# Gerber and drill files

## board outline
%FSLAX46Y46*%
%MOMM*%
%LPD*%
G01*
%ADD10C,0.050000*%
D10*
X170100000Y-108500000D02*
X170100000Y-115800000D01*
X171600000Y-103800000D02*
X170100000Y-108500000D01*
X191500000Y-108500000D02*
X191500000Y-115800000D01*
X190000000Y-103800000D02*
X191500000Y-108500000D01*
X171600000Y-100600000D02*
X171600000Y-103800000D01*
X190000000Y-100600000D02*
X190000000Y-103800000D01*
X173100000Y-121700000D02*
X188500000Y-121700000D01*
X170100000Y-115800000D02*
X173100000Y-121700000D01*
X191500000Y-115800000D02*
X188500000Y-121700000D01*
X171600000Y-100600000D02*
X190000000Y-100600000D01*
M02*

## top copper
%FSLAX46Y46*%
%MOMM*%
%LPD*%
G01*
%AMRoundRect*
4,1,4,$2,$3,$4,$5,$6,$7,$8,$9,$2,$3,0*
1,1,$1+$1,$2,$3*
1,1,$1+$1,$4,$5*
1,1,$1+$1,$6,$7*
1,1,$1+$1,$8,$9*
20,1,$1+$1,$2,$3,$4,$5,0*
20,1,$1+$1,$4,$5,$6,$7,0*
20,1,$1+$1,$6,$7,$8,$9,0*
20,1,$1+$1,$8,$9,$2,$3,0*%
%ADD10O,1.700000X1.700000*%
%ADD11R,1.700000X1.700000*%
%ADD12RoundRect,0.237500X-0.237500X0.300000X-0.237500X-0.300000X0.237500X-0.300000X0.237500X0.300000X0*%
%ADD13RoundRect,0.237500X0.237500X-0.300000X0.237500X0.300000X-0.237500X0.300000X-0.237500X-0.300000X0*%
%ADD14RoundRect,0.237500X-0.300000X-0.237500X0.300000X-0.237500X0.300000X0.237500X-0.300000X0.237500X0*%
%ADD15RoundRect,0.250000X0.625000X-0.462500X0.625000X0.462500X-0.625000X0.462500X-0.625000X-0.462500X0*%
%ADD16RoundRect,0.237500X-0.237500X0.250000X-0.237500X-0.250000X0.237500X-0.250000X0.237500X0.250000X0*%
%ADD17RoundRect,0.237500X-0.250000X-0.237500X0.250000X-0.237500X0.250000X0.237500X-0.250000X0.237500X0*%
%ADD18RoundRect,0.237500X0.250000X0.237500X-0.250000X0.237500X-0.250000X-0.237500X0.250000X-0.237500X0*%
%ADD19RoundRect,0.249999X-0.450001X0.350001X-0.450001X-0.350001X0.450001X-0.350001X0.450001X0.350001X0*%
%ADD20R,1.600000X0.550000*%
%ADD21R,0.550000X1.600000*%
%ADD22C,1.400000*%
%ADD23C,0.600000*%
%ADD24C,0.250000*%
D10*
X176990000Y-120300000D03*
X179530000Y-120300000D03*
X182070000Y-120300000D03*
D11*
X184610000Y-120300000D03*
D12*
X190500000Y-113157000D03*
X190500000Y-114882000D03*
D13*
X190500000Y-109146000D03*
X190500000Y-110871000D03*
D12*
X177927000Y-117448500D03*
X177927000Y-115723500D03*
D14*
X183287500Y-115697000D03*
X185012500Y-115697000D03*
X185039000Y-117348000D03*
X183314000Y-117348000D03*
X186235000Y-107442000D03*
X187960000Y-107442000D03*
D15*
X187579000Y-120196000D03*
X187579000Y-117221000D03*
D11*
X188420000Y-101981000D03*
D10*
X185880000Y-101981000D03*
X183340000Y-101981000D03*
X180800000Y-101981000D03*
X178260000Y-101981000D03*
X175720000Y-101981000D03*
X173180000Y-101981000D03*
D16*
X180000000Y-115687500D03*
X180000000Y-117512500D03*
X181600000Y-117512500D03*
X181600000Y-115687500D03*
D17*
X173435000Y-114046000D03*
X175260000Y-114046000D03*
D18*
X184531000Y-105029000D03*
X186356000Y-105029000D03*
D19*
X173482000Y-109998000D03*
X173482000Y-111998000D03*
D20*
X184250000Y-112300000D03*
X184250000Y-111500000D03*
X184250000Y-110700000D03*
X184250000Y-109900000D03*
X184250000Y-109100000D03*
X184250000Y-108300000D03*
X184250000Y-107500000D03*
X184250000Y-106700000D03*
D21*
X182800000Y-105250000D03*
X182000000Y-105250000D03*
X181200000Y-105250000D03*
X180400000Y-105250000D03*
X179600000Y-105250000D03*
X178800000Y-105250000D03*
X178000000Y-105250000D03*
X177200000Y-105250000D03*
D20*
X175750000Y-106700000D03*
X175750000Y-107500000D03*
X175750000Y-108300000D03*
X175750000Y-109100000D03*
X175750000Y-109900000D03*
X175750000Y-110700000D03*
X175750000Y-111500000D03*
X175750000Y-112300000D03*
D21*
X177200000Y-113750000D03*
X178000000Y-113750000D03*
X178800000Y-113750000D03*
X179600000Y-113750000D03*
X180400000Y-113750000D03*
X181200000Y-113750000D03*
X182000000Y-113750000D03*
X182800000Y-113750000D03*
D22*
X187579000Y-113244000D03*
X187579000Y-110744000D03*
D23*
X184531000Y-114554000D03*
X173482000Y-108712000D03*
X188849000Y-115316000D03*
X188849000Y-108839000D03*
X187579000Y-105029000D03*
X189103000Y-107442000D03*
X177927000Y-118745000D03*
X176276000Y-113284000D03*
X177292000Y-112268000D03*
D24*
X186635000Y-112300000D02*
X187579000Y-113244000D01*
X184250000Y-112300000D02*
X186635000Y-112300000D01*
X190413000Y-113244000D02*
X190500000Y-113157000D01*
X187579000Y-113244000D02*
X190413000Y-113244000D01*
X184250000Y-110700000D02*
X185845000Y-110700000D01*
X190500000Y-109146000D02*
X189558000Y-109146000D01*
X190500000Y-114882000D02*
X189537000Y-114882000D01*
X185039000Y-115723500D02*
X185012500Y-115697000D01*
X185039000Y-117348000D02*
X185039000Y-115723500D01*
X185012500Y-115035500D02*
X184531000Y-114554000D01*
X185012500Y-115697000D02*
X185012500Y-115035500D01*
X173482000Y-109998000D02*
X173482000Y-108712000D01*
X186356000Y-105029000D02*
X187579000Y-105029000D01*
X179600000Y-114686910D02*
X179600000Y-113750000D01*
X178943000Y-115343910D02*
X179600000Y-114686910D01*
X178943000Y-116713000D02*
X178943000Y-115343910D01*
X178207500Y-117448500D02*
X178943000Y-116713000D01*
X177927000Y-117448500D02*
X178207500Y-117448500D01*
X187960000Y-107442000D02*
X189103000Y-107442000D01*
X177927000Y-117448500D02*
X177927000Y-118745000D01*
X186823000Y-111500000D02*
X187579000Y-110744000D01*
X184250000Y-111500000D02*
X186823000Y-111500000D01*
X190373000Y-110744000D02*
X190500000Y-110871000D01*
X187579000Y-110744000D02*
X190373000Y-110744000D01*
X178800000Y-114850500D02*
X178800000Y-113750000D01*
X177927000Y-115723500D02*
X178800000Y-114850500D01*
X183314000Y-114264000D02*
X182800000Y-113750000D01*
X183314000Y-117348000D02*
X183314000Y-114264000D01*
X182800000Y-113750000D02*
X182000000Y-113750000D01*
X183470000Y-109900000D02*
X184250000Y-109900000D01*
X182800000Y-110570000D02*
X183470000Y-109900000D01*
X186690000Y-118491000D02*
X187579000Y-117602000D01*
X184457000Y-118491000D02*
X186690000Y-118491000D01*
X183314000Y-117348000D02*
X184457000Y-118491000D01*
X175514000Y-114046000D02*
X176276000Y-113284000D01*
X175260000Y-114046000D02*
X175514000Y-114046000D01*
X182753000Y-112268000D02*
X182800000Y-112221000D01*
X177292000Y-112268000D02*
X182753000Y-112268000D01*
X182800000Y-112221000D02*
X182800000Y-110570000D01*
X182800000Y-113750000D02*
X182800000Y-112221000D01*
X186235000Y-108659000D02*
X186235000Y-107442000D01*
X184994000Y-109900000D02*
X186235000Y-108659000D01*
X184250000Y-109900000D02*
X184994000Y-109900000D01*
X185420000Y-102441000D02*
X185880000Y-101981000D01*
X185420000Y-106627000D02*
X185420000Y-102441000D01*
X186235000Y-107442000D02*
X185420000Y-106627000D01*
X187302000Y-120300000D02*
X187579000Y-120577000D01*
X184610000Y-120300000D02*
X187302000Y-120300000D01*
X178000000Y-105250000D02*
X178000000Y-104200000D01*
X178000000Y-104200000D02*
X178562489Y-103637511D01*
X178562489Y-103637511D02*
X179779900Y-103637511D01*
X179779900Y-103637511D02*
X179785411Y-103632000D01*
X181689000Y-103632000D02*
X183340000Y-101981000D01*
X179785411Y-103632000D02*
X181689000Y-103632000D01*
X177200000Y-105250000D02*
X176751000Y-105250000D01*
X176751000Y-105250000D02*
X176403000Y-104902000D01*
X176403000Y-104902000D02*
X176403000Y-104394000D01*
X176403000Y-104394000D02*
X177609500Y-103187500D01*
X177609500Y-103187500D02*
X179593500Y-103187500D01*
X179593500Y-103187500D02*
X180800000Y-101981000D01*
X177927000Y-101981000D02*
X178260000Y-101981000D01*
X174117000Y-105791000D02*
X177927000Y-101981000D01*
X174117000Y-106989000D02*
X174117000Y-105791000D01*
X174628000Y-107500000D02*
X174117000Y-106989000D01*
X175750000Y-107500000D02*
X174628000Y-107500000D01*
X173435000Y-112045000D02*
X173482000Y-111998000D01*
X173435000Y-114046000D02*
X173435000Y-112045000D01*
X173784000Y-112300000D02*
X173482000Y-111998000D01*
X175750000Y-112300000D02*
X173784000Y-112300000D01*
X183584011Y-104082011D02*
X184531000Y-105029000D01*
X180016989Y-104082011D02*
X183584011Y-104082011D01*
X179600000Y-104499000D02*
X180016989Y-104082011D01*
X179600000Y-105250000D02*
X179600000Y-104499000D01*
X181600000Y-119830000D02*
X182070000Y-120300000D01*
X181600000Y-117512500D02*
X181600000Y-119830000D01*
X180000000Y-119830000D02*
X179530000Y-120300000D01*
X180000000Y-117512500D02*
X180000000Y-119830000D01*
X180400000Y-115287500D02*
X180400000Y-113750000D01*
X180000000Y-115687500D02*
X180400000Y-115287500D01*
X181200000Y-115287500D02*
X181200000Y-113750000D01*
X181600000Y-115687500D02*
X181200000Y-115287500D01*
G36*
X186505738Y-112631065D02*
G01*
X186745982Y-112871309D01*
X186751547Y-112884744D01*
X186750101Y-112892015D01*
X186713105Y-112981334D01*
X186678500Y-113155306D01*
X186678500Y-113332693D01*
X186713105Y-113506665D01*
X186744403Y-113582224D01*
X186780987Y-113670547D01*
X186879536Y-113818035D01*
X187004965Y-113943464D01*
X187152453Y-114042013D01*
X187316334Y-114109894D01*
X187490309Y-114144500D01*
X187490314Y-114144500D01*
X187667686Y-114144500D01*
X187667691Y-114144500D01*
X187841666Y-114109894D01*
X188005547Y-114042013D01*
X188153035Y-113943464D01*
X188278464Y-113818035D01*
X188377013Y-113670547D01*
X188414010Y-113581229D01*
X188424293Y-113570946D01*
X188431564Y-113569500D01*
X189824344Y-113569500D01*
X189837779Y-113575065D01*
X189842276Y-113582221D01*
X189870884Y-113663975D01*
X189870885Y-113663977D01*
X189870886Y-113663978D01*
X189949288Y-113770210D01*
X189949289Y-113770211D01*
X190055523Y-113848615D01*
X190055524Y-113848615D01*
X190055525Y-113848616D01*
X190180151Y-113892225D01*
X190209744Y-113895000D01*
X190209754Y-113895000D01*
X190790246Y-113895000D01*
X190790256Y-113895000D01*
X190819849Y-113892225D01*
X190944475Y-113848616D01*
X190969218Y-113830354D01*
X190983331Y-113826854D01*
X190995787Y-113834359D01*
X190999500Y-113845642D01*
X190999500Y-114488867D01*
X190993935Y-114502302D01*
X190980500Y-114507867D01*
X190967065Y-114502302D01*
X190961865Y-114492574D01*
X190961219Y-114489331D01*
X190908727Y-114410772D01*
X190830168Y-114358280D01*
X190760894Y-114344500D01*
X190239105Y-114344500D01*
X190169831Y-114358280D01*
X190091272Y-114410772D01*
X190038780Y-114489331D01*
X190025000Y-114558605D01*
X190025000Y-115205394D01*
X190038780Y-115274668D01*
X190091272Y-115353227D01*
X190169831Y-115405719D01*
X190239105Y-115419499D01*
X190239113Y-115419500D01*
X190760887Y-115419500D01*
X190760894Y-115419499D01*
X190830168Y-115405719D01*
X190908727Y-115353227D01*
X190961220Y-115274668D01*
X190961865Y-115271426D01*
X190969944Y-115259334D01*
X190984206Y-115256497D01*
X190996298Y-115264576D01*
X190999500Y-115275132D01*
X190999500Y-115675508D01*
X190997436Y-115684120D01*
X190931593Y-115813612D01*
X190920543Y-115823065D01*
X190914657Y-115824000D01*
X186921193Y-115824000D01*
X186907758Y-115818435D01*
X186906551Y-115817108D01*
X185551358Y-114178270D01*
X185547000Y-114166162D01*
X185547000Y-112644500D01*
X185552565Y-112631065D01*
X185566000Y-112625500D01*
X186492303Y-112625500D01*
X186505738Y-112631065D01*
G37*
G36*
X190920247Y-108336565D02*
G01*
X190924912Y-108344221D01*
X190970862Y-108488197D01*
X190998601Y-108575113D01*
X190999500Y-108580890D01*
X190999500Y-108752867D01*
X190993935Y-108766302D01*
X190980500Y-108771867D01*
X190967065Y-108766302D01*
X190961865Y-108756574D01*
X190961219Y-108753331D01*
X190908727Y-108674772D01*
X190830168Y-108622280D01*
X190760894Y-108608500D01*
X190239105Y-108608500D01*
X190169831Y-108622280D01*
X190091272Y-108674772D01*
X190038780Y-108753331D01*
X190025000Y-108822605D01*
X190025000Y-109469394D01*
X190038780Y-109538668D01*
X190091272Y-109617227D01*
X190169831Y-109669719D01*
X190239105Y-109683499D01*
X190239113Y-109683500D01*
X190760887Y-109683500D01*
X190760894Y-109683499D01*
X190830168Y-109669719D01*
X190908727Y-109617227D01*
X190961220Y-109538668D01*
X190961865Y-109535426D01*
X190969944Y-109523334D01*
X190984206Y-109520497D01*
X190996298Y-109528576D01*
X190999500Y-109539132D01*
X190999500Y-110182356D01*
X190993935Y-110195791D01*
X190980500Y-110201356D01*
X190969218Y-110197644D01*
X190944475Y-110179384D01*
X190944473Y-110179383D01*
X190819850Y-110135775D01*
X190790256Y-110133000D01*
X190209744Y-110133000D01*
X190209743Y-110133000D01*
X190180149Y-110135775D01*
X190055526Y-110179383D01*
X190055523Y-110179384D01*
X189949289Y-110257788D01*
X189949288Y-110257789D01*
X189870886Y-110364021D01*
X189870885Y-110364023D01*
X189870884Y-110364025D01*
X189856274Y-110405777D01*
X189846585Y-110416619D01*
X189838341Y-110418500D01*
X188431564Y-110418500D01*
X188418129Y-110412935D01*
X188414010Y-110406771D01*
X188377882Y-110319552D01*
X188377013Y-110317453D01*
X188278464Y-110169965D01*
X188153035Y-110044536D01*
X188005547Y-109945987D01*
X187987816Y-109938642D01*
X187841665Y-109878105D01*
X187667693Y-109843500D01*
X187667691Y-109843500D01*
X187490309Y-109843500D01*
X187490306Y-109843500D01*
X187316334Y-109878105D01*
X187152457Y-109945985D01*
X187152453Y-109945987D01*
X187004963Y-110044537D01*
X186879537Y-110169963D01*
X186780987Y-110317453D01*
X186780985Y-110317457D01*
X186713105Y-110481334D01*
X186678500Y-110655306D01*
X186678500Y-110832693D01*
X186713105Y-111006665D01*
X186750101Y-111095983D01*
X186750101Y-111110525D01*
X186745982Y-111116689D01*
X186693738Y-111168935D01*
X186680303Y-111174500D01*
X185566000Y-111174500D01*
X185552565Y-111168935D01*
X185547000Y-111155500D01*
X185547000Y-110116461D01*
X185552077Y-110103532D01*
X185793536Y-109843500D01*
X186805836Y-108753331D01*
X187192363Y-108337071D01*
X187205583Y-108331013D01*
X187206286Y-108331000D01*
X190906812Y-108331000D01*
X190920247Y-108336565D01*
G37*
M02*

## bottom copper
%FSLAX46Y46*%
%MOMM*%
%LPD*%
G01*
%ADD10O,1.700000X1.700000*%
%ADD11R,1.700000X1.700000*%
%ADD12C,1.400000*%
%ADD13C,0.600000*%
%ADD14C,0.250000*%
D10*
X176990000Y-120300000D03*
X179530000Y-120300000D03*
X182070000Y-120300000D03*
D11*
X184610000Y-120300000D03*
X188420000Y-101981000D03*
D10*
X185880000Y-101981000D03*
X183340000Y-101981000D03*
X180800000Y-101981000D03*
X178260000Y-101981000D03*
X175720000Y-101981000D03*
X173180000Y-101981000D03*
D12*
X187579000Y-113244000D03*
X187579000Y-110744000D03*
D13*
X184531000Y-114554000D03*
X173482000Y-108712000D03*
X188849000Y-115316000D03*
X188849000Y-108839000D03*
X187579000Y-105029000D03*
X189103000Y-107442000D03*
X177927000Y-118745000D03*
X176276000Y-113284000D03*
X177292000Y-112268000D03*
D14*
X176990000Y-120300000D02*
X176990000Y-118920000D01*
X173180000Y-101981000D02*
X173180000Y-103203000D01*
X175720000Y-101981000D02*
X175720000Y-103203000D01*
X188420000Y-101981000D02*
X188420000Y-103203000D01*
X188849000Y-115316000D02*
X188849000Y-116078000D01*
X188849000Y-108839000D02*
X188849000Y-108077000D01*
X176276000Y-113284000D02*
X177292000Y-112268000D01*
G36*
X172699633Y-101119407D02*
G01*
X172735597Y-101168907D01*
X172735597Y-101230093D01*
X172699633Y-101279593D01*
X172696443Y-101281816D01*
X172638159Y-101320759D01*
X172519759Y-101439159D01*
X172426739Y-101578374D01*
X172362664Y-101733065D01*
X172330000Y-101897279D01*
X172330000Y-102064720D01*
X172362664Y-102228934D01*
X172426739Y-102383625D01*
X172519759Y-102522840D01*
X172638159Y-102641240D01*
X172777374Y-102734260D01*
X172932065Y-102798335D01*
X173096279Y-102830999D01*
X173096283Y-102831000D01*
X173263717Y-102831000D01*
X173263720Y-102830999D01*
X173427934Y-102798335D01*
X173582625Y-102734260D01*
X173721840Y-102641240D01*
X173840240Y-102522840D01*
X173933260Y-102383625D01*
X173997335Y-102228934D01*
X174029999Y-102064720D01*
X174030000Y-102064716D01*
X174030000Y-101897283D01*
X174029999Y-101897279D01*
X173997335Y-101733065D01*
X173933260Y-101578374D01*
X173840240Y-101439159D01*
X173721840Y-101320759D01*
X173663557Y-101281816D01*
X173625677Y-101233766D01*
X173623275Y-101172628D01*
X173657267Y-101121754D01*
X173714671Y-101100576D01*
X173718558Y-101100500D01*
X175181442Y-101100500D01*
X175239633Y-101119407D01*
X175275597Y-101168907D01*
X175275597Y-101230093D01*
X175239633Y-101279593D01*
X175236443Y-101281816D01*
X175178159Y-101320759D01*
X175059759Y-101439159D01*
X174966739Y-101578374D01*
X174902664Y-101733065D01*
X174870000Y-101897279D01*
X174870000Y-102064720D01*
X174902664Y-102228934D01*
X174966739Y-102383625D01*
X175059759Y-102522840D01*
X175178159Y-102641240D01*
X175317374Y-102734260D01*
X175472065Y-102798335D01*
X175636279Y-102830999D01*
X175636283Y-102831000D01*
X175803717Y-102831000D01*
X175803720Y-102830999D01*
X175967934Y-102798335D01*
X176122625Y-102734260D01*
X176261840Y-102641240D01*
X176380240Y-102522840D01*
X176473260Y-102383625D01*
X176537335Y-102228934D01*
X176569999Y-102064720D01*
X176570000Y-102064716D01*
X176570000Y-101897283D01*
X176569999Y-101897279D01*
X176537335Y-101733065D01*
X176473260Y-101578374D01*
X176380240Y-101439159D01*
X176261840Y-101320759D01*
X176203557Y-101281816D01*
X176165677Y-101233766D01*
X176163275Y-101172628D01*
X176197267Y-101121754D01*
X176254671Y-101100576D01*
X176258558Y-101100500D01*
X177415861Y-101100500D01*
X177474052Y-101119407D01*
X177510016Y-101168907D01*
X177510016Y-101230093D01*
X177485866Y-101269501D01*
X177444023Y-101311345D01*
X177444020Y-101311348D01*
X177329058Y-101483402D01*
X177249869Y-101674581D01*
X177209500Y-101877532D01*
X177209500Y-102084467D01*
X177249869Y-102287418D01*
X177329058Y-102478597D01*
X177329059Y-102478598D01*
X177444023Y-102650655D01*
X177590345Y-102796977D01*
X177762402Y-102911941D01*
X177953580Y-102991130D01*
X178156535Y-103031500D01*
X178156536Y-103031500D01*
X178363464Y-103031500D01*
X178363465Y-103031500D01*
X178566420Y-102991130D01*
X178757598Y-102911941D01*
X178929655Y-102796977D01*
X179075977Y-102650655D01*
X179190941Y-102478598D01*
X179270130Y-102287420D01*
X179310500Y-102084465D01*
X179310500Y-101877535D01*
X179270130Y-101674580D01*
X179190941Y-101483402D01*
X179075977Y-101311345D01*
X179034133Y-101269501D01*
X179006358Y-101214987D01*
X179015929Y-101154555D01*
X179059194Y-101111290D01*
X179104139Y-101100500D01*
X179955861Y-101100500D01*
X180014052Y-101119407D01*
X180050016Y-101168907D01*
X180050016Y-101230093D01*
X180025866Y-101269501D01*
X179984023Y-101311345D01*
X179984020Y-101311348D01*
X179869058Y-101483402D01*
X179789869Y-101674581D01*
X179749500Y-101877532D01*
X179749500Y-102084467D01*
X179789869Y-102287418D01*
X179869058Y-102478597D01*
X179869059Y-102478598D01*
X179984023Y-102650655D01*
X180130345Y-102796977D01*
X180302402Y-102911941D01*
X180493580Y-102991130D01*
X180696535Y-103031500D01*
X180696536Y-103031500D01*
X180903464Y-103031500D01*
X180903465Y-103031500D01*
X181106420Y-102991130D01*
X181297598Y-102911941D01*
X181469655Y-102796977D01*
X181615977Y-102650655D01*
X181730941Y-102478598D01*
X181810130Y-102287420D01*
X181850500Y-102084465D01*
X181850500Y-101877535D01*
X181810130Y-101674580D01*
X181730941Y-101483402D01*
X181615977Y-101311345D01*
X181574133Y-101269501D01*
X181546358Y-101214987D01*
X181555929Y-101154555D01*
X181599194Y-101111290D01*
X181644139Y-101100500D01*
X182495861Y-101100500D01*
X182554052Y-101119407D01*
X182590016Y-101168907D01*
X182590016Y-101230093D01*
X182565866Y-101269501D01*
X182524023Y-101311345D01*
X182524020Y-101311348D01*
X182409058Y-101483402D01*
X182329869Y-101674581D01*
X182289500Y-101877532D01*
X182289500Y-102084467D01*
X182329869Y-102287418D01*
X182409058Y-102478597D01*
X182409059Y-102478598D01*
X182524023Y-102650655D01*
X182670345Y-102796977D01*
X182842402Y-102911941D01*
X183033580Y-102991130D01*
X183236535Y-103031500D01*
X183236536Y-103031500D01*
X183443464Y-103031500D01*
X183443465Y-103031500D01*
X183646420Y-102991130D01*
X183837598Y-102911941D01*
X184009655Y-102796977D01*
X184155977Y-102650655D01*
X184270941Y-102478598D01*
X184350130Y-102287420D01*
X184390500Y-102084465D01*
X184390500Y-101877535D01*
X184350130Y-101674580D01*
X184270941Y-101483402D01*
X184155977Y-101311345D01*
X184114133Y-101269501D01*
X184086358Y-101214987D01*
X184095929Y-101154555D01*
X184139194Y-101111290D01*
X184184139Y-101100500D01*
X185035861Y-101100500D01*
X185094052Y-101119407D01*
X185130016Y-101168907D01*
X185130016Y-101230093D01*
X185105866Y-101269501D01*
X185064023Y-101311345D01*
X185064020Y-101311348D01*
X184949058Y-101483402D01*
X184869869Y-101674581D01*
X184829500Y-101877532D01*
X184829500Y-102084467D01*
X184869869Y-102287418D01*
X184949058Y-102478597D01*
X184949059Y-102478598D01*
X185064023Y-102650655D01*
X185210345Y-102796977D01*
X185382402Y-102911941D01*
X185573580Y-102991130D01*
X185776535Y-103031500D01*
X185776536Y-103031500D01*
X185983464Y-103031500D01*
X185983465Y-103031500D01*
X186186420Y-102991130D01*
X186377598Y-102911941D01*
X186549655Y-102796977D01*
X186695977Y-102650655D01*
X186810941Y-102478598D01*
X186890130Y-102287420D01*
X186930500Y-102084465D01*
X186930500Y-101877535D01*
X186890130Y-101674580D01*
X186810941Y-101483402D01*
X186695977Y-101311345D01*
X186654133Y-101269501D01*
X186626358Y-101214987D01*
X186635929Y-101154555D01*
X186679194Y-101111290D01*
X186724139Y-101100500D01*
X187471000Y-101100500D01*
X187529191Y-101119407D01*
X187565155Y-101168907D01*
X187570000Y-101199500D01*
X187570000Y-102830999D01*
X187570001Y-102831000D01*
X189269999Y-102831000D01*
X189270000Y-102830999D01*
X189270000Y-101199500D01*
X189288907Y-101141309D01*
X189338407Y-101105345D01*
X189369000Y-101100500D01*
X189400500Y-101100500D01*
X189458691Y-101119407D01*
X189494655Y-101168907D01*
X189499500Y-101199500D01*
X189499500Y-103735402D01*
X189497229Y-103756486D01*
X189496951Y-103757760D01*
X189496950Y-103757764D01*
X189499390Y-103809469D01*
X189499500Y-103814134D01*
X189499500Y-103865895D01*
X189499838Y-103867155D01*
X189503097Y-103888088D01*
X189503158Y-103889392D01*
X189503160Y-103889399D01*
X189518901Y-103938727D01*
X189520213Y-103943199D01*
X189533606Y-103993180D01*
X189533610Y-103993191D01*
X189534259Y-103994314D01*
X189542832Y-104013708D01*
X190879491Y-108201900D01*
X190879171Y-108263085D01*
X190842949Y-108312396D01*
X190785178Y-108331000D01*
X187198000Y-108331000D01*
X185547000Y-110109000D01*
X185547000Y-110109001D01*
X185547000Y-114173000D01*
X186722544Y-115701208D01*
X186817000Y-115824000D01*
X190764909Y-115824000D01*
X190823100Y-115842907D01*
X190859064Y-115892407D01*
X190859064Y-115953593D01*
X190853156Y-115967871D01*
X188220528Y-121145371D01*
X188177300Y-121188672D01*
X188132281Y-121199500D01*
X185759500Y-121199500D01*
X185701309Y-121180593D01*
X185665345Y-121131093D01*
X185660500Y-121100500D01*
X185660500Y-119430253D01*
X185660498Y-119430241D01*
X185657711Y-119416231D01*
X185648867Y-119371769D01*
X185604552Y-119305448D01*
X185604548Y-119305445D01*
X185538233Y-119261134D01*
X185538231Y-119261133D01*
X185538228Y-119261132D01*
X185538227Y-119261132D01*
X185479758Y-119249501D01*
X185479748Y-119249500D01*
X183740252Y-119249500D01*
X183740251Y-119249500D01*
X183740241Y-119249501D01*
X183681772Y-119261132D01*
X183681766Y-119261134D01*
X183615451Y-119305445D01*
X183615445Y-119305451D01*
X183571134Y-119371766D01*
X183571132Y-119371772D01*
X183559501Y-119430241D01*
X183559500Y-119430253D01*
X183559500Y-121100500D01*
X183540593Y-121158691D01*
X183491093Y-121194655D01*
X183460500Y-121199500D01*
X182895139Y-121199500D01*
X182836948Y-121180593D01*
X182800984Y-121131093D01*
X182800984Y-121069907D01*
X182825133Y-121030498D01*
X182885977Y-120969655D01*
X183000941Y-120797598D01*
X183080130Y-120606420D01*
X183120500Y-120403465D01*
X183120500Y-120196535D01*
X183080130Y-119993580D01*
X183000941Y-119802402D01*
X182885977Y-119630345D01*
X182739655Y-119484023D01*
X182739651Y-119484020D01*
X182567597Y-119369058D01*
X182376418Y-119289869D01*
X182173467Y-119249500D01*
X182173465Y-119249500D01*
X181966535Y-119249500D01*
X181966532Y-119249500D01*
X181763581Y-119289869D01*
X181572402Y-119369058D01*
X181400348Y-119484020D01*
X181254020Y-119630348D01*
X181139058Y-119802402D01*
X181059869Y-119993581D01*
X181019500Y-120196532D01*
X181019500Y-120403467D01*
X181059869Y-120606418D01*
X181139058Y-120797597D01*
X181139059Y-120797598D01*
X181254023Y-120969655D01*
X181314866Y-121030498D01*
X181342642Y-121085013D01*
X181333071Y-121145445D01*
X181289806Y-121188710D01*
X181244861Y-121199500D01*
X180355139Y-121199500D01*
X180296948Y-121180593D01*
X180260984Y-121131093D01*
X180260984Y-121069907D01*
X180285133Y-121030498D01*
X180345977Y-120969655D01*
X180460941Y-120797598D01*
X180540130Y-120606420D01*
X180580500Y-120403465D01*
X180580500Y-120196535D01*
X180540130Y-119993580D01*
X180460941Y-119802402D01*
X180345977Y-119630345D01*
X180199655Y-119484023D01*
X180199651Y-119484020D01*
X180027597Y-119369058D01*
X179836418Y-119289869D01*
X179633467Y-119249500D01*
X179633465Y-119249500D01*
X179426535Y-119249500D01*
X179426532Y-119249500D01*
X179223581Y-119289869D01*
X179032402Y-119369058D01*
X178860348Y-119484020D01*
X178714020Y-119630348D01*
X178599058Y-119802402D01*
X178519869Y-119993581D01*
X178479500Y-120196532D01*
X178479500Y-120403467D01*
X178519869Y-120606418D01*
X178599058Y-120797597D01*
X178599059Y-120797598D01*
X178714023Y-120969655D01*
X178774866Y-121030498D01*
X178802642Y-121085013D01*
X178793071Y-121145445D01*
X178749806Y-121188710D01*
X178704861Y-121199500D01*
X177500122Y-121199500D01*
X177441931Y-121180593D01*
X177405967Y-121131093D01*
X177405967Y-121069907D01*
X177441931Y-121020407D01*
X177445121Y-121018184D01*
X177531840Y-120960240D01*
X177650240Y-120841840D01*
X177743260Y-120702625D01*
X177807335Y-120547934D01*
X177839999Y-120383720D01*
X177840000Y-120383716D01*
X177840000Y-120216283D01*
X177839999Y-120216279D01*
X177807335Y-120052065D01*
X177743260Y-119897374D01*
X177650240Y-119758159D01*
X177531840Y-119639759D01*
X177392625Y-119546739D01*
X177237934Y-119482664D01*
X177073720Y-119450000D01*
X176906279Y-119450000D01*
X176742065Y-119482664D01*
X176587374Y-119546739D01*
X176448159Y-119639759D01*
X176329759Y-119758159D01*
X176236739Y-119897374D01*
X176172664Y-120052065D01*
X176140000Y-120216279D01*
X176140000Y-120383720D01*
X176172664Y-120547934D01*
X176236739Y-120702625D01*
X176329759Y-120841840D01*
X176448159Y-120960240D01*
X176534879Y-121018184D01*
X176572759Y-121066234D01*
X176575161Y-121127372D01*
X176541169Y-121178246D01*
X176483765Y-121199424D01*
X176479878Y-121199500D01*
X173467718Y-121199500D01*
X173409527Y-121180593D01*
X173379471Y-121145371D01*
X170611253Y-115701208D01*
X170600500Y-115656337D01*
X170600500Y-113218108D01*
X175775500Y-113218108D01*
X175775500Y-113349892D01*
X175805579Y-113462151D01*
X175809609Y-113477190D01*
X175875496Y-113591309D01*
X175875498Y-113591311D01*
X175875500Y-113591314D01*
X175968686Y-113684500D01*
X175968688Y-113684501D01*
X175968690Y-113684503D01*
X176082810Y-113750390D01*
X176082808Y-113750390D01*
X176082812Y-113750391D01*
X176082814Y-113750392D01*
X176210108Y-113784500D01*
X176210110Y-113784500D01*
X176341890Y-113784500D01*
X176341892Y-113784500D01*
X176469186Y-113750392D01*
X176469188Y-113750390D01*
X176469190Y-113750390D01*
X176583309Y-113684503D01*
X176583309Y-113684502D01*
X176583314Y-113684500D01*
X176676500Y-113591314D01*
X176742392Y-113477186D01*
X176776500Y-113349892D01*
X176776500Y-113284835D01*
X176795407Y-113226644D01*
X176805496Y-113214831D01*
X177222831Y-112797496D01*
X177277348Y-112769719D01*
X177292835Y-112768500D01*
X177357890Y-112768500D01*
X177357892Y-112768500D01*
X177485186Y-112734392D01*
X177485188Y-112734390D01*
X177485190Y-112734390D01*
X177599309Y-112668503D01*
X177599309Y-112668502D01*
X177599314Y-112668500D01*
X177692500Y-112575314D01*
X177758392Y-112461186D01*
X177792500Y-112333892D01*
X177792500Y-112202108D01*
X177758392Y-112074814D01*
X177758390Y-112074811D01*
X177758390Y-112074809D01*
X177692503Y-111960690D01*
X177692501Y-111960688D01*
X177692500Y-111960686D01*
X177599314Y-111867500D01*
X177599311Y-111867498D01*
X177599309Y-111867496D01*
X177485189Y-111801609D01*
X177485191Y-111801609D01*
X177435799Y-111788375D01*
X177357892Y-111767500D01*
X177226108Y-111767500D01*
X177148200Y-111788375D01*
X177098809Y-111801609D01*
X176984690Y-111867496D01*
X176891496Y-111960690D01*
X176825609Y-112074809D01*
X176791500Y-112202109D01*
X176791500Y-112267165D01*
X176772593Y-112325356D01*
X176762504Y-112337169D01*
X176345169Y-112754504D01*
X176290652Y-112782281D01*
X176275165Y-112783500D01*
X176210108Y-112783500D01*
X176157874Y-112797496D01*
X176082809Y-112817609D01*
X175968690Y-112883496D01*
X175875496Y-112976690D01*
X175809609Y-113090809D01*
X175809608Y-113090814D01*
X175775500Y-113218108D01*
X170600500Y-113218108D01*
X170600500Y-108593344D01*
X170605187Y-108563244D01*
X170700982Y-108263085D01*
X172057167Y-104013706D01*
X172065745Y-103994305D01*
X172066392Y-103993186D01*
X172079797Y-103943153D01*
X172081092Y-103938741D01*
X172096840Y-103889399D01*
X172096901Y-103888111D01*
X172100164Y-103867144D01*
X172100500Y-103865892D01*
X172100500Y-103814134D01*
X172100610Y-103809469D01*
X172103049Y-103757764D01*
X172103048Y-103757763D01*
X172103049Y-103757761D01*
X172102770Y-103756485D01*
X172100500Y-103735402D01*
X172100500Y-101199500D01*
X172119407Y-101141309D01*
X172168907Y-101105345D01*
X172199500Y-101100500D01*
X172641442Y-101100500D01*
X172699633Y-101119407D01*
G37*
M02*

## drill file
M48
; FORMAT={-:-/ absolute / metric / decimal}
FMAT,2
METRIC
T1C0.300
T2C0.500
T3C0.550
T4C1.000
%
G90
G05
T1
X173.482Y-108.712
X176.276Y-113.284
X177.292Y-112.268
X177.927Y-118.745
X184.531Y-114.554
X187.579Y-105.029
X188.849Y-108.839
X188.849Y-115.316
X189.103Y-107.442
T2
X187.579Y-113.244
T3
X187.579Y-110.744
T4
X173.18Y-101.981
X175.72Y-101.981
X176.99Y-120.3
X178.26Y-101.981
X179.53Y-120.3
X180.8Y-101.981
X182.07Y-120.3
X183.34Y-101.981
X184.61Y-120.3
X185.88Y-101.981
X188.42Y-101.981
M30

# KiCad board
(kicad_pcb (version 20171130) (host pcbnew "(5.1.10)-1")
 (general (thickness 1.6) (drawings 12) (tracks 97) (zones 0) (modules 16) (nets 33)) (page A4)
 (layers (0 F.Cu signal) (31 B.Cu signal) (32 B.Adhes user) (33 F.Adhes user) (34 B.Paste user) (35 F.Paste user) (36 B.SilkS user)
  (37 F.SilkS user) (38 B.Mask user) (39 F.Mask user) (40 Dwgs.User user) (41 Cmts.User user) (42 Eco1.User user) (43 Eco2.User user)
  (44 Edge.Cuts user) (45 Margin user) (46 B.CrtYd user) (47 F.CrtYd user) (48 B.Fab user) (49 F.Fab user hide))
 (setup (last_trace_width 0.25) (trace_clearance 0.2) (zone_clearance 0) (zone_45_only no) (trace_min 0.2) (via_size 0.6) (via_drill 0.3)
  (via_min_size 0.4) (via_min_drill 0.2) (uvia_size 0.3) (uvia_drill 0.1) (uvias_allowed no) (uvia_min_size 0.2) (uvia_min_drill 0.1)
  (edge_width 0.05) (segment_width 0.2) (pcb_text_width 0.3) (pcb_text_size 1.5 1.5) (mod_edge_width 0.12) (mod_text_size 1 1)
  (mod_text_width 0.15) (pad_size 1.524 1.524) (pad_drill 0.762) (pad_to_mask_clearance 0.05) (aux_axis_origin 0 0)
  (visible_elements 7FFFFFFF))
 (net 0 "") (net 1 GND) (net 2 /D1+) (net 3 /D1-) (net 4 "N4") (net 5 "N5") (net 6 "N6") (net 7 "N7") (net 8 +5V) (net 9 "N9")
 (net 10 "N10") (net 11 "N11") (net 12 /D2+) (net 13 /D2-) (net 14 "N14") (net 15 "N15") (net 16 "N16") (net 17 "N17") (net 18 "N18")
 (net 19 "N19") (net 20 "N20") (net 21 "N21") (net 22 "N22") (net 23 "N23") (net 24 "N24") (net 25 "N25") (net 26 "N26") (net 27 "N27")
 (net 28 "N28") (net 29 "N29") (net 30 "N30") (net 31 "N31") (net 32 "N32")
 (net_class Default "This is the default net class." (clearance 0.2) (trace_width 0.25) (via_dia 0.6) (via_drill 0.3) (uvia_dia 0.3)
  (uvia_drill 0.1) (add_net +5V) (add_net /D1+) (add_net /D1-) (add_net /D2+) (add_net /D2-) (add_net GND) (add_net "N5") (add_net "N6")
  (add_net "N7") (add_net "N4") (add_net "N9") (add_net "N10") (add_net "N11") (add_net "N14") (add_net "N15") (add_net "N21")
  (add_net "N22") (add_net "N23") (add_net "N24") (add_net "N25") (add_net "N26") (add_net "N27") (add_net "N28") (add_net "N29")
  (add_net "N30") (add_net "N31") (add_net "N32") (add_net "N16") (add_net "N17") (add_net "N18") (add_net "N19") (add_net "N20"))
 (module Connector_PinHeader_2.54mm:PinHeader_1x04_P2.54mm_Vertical (layer F.Cu) (at 184.61 120.3 270)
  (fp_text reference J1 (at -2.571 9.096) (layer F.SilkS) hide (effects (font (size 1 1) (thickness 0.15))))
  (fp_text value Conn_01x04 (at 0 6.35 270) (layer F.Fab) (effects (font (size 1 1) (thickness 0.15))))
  (pad 4 thru_hole oval (at 0 7.62 270) (size 1.7 1.7) (drill 1) (layers *.Cu *.Mask) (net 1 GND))
  (pad 3 thru_hole oval (at 0 5.08 270) (size 1.7 1.7) (drill 1) (layers *.Cu *.Mask) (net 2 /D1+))
  (pad 2 thru_hole oval (at 0 2.54 270) (size 1.7 1.7) (drill 1) (layers *.Cu *.Mask) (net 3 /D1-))
  (pad 1 thru_hole rect (at 0 0 270) (size 1.7 1.7) (drill 1) (layers *.Cu *.Mask) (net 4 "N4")))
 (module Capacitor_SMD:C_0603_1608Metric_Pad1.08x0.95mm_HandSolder (layer F.Cu) (at 190.5 114.0195 270)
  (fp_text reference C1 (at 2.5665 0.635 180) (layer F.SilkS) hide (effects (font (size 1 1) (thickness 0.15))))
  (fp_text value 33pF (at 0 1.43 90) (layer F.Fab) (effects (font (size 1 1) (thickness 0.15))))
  (pad 1 smd roundrect (at -0.8625 0 270) (size 1.075 0.95) (layers F.Cu F.Paste F.Mask) (roundrect_rratio 0.25) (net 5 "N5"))
  (pad 2 smd roundrect (at 0.8625 0 270) (size 1.075 0.95) (layers F.Cu F.Paste F.Mask) (roundrect_rratio 0.25) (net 1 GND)))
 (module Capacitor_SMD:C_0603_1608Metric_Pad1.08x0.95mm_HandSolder (layer F.Cu) (at 190.5 110.0085 90)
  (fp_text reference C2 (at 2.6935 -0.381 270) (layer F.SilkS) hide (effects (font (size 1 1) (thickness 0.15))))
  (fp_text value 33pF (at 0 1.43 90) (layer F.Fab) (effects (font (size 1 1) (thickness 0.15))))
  (pad 2 smd roundrect (at 0.8625 0 90) (size 1.075 0.95) (layers F.Cu F.Paste F.Mask) (roundrect_rratio 0.25) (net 1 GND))
  (pad 1 smd roundrect (at -0.8625 0 90) (size 1.075 0.95) (layers F.Cu F.Paste F.Mask) (roundrect_rratio 0.25) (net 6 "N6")))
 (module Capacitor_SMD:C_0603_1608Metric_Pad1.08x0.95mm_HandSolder (layer F.Cu) (at 177.927 116.586 270)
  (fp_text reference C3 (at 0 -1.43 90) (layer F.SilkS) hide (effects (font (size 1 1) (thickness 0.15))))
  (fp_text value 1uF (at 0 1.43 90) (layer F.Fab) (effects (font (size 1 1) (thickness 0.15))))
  (pad 2 smd roundrect (at 0.8625 0 270) (size 1.075 0.95) (layers F.Cu F.Paste F.Mask) (roundrect_rratio 0.25) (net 1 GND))
  (pad 1 smd roundrect (at -0.8625 0 270) (size 1.075 0.95) (layers F.Cu F.Paste F.Mask) (roundrect_rratio 0.25) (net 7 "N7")))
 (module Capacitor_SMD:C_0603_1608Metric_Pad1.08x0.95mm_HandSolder (layer F.Cu) (at 184.15 115.697)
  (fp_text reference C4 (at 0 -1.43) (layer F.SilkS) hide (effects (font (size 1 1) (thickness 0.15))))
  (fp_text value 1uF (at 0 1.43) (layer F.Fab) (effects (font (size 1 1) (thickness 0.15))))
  (pad 1 smd roundrect (at -0.8625 0) (size 1.075 0.95) (layers F.Cu F.Paste F.Mask) (roundrect_rratio 0.25) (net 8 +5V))
  (pad 2 smd roundrect (at 0.8625 0) (size 1.075 0.95) (layers F.Cu F.Paste F.Mask) (roundrect_rratio 0.25) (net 1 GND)))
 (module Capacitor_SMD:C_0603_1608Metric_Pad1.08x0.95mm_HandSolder (layer F.Cu) (at 184.1765 117.348)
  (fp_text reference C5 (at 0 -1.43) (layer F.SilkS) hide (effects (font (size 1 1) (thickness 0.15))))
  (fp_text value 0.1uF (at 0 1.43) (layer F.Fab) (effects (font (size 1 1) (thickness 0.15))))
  (pad 2 smd roundrect (at 0.8625 0) (size 1.075 0.95) (layers F.Cu F.Paste F.Mask) (roundrect_rratio 0.25) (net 1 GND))
  (pad 1 smd roundrect (at -0.8625 0) (size 1.075 0.95) (layers F.Cu F.Paste F.Mask) (roundrect_rratio 0.25) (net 8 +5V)))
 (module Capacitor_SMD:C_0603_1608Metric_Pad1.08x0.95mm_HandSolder (layer F.Cu) (at 187.0975 107.442)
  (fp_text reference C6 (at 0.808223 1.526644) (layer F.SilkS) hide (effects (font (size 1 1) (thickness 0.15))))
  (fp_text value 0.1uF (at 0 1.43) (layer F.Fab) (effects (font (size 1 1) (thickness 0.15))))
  (pad 1 smd roundrect (at -0.8625 0) (size 1.075 0.95) (layers F.Cu F.Paste F.Mask) (roundrect_rratio 0.25) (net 8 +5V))
  (pad 2 smd roundrect (at 0.8625 0) (size 1.075 0.95) (layers F.Cu F.Paste F.Mask) (roundrect_rratio 0.25) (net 1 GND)))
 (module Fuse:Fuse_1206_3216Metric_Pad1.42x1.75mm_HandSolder (layer F.Cu) (at 187.579 118.7085 90)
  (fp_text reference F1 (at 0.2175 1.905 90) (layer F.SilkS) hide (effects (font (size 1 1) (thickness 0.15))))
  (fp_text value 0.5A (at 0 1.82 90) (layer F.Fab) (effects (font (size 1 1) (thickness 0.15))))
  (pad 1 smd roundrect (at -1.4875 0 90) (size 1.425 1.75) (layers F.Cu F.Paste F.Mask) (roundrect_rratio 0.1754385964912281) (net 4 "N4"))
  (pad 2 smd roundrect (at 1.4875 0 90) (size 1.425 1.75) (layers F.Cu F.Paste F.Mask) (roundrect_rratio 0.1754385964912281) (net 8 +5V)))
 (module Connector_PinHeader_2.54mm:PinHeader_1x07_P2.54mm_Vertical (layer F.Cu) (at 188.42 101.981 270)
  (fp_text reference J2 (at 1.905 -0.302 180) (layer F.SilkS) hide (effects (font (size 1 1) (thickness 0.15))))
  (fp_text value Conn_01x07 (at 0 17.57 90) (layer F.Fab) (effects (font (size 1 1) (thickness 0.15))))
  (pad 1 thru_hole rect (at 0 0 270) (size 1.7 1.7) (drill 1) (layers *.Cu *.Mask) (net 1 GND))
  (pad 2 thru_hole oval (at 0 2.54 270) (size 1.7 1.7) (drill 1) (layers *.Cu *.Mask) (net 8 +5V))
  (pad 3 thru_hole oval (at 0 5.08 270) (size 1.7 1.7) (drill 1) (layers *.Cu *.Mask) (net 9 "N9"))
  (pad 4 thru_hole oval (at 0 7.62 270) (size 1.7 1.7) (drill 1) (layers *.Cu *.Mask) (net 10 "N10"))
  (pad 5 thru_hole oval (at 0 10.16 270) (size 1.7 1.7) (drill 1) (layers *.Cu *.Mask) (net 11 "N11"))
  (pad 6 thru_hole oval (at 0 12.7 270) (size 1.7 1.7) (drill 1) (layers *.Cu *.Mask) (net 1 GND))
  (pad 7 thru_hole oval (at 0 15.24 270) (size 1.7 1.7) (drill 1) (layers *.Cu *.Mask) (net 1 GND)))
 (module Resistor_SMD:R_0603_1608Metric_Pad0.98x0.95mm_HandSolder (layer F.Cu) (at 180 116.6 270)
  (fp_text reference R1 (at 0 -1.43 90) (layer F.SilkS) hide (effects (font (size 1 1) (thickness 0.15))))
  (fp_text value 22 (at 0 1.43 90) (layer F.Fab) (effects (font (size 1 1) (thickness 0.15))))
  (pad 1 smd roundrect (at -0.9125 0 270) (size 0.975 0.95) (layers F.Cu F.Paste F.Mask) (roundrect_rratio 0.25) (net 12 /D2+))
  (pad 2 smd roundrect (at 0.9125 0 270) (size 0.975 0.95) (layers F.Cu F.Paste F.Mask) (roundrect_rratio 0.25) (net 2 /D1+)))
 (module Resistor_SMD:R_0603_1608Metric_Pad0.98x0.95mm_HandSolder (layer F.Cu) (at 181.6 116.6 270)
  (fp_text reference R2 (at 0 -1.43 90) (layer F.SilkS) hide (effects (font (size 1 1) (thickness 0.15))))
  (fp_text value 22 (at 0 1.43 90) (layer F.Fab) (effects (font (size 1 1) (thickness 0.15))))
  (pad 2 smd roundrect (at 0.9125 0 270) (size 0.975 0.95) (layers F.Cu F.Paste F.Mask) (roundrect_rratio 0.25) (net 3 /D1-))
  (pad 1 smd roundrect (at -0.9125 0 270) (size 0.975 0.95) (layers F.Cu F.Paste F.Mask) (roundrect_rratio 0.25) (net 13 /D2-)))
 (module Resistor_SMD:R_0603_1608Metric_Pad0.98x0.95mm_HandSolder (layer F.Cu) (at 174.3475 114.046)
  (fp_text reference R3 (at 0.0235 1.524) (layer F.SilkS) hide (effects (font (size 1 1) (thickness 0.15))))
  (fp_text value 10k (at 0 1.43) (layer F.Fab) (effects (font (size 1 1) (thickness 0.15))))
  (pad 1 smd roundrect (at -0.9125 0) (size 0.975 0.95) (layers F.Cu F.Paste F.Mask) (roundrect_rratio 0.25) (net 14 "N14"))
  (pad 2 smd roundrect (at 0.9125 0) (size 0.975 0.95) (layers F.Cu F.Paste F.Mask) (roundrect_rratio 0.25) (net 8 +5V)))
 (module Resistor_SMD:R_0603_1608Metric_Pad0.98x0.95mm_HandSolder (layer F.Cu) (at 185.4435 105.029 180)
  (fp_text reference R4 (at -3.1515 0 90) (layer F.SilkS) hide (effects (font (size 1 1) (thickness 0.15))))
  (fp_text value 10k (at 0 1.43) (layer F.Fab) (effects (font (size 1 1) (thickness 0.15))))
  (pad 2 smd roundrect (at 0.9125 0 180) (size 0.975 0.95) (layers F.Cu F.Paste F.Mask) (roundrect_rratio 0.25) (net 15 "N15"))
  (pad 1 smd roundrect (at -0.9125 0 180) (size 0.975 0.95) (layers F.Cu F.Paste F.Mask) (roundrect_rratio 0.25) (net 1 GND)))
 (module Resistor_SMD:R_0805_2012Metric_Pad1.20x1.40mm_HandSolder (layer F.Cu) (at 173.482 110.998 270)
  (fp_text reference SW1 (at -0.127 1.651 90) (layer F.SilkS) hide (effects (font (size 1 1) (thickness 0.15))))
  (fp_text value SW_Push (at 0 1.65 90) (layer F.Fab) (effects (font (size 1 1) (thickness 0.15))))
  (pad 1 smd roundrect (at -1 0 270) (size 1.2 1.4) (layers F.Cu F.Paste F.Mask) (roundrect_rratio 0.2083325) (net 1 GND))
  (pad 2 smd roundrect (at 1 0 270) (size 1.2 1.4) (layers F.Cu F.Paste F.Mask) (roundrect_rratio 0.2083325) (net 14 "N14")))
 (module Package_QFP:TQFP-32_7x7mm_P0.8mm (layer F.Cu) (at 180 109.5 180)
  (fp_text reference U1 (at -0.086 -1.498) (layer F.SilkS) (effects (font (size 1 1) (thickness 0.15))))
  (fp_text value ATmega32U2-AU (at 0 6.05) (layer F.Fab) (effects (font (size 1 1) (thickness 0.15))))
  (pad 1 smd rect (at -4.25 -2.8 180) (size 1.6 0.55) (layers F.Cu F.Paste F.Mask) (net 5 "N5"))
  (pad 2 smd rect (at -4.25 -2 180) (size 1.6 0.55) (layers F.Cu F.Paste F.Mask) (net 6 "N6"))
  (pad 3 smd rect (at -4.25 -1.2 180) (size 1.6 0.55) (layers F.Cu F.Paste F.Mask) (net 1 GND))
  (pad 4 smd rect (at -4.25 -0.4 180) (size 1.6 0.55) (layers F.Cu F.Paste F.Mask) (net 8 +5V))
  (pad 5 smd rect (at -4.25 0.4 180) (size 1.6 0.55) (layers F.Cu F.Paste F.Mask) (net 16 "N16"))
  (pad 6 smd rect (at -4.25 1.2 180) (size 1.6 0.55) (layers F.Cu F.Paste F.Mask) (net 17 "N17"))
  (pad 7 smd rect (at -4.25 2 180) (size 1.6 0.55) (layers F.Cu F.Paste F.Mask) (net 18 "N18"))
  (pad 8 smd rect (at -4.25 2.8 180) (size 1.6 0.55) (layers F.Cu F.Paste F.Mask) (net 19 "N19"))
  (pad 9 smd rect (at -2.8 4.25 270) (size 1.6 0.55) (layers F.Cu F.Paste F.Mask) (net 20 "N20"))
  (pad 10 smd rect (at -2 4.25 270) (size 1.6 0.55) (layers F.Cu F.Paste F.Mask) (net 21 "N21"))
  (pad 11 smd rect (at -1.2 4.25 270) (size 1.6 0.55) (layers F.Cu F.Paste F.Mask) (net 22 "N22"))
  (pad 12 smd rect (at -0.4 4.25 270) (size 1.6 0.55) (layers F.Cu F.Paste F.Mask) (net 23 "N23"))
  (pad 13 smd rect (at 0.4 4.25 270) (size 1.6 0.55) (layers F.Cu F.Paste F.Mask) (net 15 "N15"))
  (pad 14 smd rect (at 1.2 4.25 270) (size 1.6 0.55) (layers F.Cu F.Paste F.Mask) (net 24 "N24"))
  (pad 15 smd rect (at 2 4.25 270) (size 1.6 0.55) (layers F.Cu F.Paste F.Mask) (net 9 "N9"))
  (pad 16 smd rect (at 2.8 4.25 270) (size 1.6 0.55) (layers F.Cu F.Paste F.Mask) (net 10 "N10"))
  (pad 17 smd rect (at 4.25 2.8 180) (size 1.6 0.55) (layers F.Cu F.Paste F.Mask) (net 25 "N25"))
  (pad 18 smd rect (at 4.25 2 180) (size 1.6 0.55) (layers F.Cu F.Paste F.Mask) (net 11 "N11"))
  (pad 19 smd rect (at 4.25 1.2 180) (size 1.6 0.55) (layers F.Cu F.Paste F.Mask) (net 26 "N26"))
  (pad 20 smd rect (at 4.25 0.4 180) (size 1.6 0.55) (layers F.Cu F.Paste F.Mask) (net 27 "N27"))
  (pad 21 smd rect (at 4.25 -0.4 180) (size 1.6 0.55) (layers F.Cu F.Paste F.Mask) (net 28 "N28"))
  (pad 22 smd rect (at 4.25 -1.2 180) (size 1.6 0.55) (layers F.Cu F.Paste F.Mask) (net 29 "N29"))
  (pad 23 smd rect (at 4.25 -2 180) (size 1.6 0.55) (layers F.Cu F.Paste F.Mask) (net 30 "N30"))
  (pad 24 smd rect (at 4.25 -2.8 180) (size 1.6 0.55) (layers F.Cu F.Paste F.Mask) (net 14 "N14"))
  (pad 25 smd rect (at 2.8 -4.25 270) (size 1.6 0.55) (layers F.Cu F.Paste F.Mask) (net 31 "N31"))
  (pad 26 smd rect (at 2 -4.25 270) (size 1.6 0.55) (layers F.Cu F.Paste F.Mask) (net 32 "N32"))
  (pad 27 smd rect (at 1.2 -4.25 270) (size 1.6 0.55) (layers F.Cu F.Paste F.Mask) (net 7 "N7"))
  (pad 28 smd rect (at 0.4 -4.25 270) (size 1.6 0.55) (layers F.Cu F.Paste F.Mask) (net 1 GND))
  (pad 29 smd rect (at -0.4 -4.25 270) (size 1.6 0.55) (layers F.Cu F.Paste F.Mask) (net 12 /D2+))
  (pad 30 smd rect (at -1.2 -4.25 270) (size 1.6 0.55) (layers F.Cu F.Paste F.Mask) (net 13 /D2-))
  (pad 31 smd rect (at -2 -4.25 270) (size 1.6 0.55) (layers F.Cu F.Paste F.Mask) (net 8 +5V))
  (pad 32 smd rect (at -2.8 -4.25 270) (size 1.6 0.55) (layers F.Cu F.Paste F.Mask) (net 8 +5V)))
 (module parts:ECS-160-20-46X (layer F.Cu) (at 187.579 111.994 90)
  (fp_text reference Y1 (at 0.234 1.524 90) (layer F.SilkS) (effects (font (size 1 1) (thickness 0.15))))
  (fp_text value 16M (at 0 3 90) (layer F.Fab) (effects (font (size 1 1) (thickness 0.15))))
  (pad 1 thru_hole circle (at -1.25 0 90) (size 1.4 1.4) (drill 0.5) (layers *.Cu B.Mask) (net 5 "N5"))
  (pad 2 thru_hole circle (at 1.25 0 90) (size 1.4 1.4) (drill 0.55) (layers *.Cu B.Mask) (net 6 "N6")))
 (gr_line (start 170.1 108.5) (end 170.1 115.8) (layer Edge.Cuts) (width 0.05))
 (gr_line (start 171.6 103.8) (end 170.1 108.5) (layer Edge.Cuts) (width 0.05))
 (gr_line (start 191.5 108.5) (end 191.5 115.8) (layer Edge.Cuts) (width 0.05))
 (gr_line (start 190 103.8) (end 191.5 108.5) (layer Edge.Cuts) (width 0.05))
 (gr_line (start 171.6 100.6) (end 171.6 103.8) (layer Edge.Cuts) (width 0.05))
 (gr_line (start 190 100.6) (end 190 103.8) (layer Edge.Cuts) (width 0.05))
 (gr_line (start 173.1 121.7) (end 188.5 121.7) (layer Edge.Cuts) (width 0.05))
 (gr_line (start 170.1 115.8) (end 173.1 121.7) (layer Edge.Cuts) (width 0.05))
 (gr_line (start 191.5 115.8) (end 188.5 121.7) (layer Edge.Cuts) (width 0.05))
 (gr_line (start 171.6 100.6) (end 190 100.6) (layer Edge.Cuts) (width 0.05))
 (segment (start 186.635 112.3) (end 187.579 113.244) (width 0.25) (layer F.Cu) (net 5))
 (segment (start 184.25 112.3) (end 186.635 112.3) (width 0.25) (layer F.Cu) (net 5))
 (segment (start 190.413 113.244) (end 190.5 113.157) (width 0.25) (layer F.Cu) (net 5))
 (segment (start 187.579 113.244) (end 190.413 113.244) (width 0.25) (layer F.Cu) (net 5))
 (segment (start 184.25 110.7) (end 185.845 110.7) (width 0.25) (layer F.Cu) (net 1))
 (segment (start 190.5 109.146) (end 189.558 109.146) (width 0.25) (layer F.Cu) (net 1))
 (segment (start 190.5 114.882) (end 189.537 114.882) (width 0.25) (layer F.Cu) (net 1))
 (segment (start 176.99 120.3) (end 176.99 118.92) (width 0.25) (layer B.Cu) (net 1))
 (segment (start 185.039 115.7235) (end 185.0125 115.697) (width 0.25) (layer F.Cu) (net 1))
 (segment (start 185.039 117.348) (end 185.039 115.7235) (width 0.25) (layer F.Cu) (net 1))
 (via (at 184.531 114.554) (size 0.6) (drill 0.3) (layers F.Cu B.Cu) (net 1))
 (segment (start 185.0125 115.0355) (end 184.531 114.554) (width 0.25) (layer F.Cu) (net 1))
 (segment (start 185.0125 115.697) (end 185.0125 115.0355) (width 0.25) (layer F.Cu) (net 1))
 (via (at 173.482 108.712) (size 0.6) (drill 0.3) (layers F.Cu B.Cu) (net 1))
 (segment (start 173.482 109.998) (end 173.482 108.712) (width 0.25) (layer F.Cu) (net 1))
 (segment (start 173.18 101.981) (end 173.18 103.203) (width 0.25) (layer B.Cu) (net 1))
 (segment (start 175.72 101.981) (end 175.72 103.203) (width 0.25) (layer B.Cu) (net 1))
 (segment (start 188.42 101.981) (end 188.42 103.203) (width 0.25) (layer B.Cu) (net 1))
 (via (at 188.849 115.316) (size 0.6) (drill 0.3) (layers F.Cu B.Cu) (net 1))
 (segment (start 188.849 115.316) (end 188.849 116.078) (width 0.25) (layer B.Cu) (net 1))
 (via (at 188.849 108.839) (size 0.6) (drill 0.3) (layers F.Cu B.Cu) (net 1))
 (segment (start 188.849 108.839) (end 188.849 108.077) (width 0.25) (layer B.Cu) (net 1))
 (via (at 187.579 105.029) (size 0.6) (drill 0.3) (layers F.Cu B.Cu) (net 1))
 (segment (start 186.356 105.029) (end 187.579 105.029) (width 0.25) (layer F.Cu) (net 1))
 (segment (start 179.6 114.68691) (end 179.6 113.75) (width 0.25) (layer F.Cu) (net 1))
 (segment (start 178.943 115.34391) (end 179.6 114.68691) (width 0.25) (layer F.Cu) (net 1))
 (segment (start 178.943 116.713) (end 178.943 115.34391) (width 0.25) (layer F.Cu) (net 1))
 (segment (start 178.2075 117.4485) (end 178.943 116.713) (width 0.25) (layer F.Cu) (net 1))
 (segment (start 177.927 117.4485) (end 178.2075 117.4485) (width 0.25) (layer F.Cu) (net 1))
 (via (at 189.103 107.442) (size 0.6) (drill 0.3) (layers F.Cu B.Cu) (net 1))
 (segment (start 187.96 107.442) (end 189.103 107.442) (width 0.25) (layer F.Cu) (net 1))
 (via (at 177.927 118.745) (size 0.6) (drill 0.3) (layers F.Cu B.Cu) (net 1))
 (segment (start 177.927 117.4485) (end 177.927 118.745) (width 0.25) (layer F.Cu) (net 1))
 (segment (start 186.823 111.5) (end 187.579 110.744) (width 0.25) (layer F.Cu) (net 6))
 (segment (start 184.25 111.5) (end 186.823 111.5) (width 0.25) (layer F.Cu) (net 6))
 (segment (start 190.373 110.744) (end 190.5 110.871) (width 0.25) (layer F.Cu) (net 6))
 (segment (start 187.579 110.744) (end 190.373 110.744) (width 0.25) (layer F.Cu) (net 6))
 (segment (start 178.8 114.8505) (end 178.8 113.75) (width 0.25) (layer F.Cu) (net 7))
 (segment (start 177.927 115.7235) (end 178.8 114.8505) (width 0.25) (layer F.Cu) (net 7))
 (segment (start 183.314 114.264) (end 182.8 113.75) (width 0.25) (layer F.Cu) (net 8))
 (segment (start 183.314 117.348) (end 183.314 114.264) (width 0.25) (layer F.Cu) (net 8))
 (segment (start 182.8 113.75) (end 182 113.75) (width 0.25) (layer F.Cu) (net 8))
 (segment (start 183.47 109.9) (end 184.25 109.9) (width 0.25) (layer F.Cu) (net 8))
 (segment (start 182.8 110.57) (end 183.47 109.9) (width 0.25) (layer F.Cu) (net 8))
 (segment (start 186.69 118.491) (end 187.579 117.602) (width 0.25) (layer F.Cu) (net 8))
 (segment (start 184.457 118.491) (end 186.69 118.491) (width 0.25) (layer F.Cu) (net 8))
 (segment (start 183.314 117.348) (end 184.457 118.491) (width 0.25) (layer F.Cu) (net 8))
 (via (at 176.276 113.284) (size 0.6) (drill 0.3) (layers F.Cu B.Cu) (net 8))
 (segment (start 175.514 114.046) (end 176.276 113.284) (width 0.25) (layer F.Cu) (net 8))
 (segment (start 175.26 114.046) (end 175.514 114.046) (width 0.25) (layer F.Cu) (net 8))
 (via (at 177.292 112.268) (size 0.6) (drill 0.3) (layers F.Cu B.Cu) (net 8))
 (segment (start 176.276 113.284) (end 177.292 112.268) (width 0.25) (layer B.Cu) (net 8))
 (segment (start 182.753 112.268) (end 182.8 112.221) (width 0.25) (layer F.Cu) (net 8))
 (segment (start 177.292 112.268) (end 182.753 112.268) (width 0.25) (layer F.Cu) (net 8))
 (segment (start 182.8 112.221) (end 182.8 110.57) (width 0.25) (layer F.Cu) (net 8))
 (segment (start 182.8 113.75) (end 182.8 112.221) (width 0.25) (layer F.Cu) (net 8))
 (segment (start 186.235 108.659) (end 186.235 107.442) (width 0.25) (layer F.Cu) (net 8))
 (segment (start 184.994 109.9) (end 186.235 108.659) (width 0.25) (layer F.Cu) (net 8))
 (segment (start 184.25 109.9) (end 184.994 109.9) (width 0.25) (layer F.Cu) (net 8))
 (segment (start 185.42 102.441) (end 185.88 101.981) (width 0.25) (layer F.Cu) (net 8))
 (segment (start 185.42 106.627) (end 185.42 102.441) (width 0.25) (layer F.Cu) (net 8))
 (segment (start 186.235 107.442) (end 185.42 106.627) (width 0.25) (layer F.Cu) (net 8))
 (segment (start 187.302 120.3) (end 187.579 120.577) (width 0.25) (layer F.Cu) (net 4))
 (segment (start 184.61 120.3) (end 187.302 120.3) (width 0.25) (layer F.Cu) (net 4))
 (segment (start 178 105.25) (end 178 104.2) (width 0.25) (layer F.Cu) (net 9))
 (segment (start 178 104.2) (end 178.562489 103.637511) (width 0.25) (layer F.Cu) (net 9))
 (segment (start 178.562489 103.637511) (end 179.7799 103.637511) (width 0.25) (layer F.Cu) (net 9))
 (segment (start 179.7799 103.637511) (end 179.785411 103.632) (width 0.25) (layer F.Cu) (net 9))
 (segment (start 181.689 103.632) (end 183.34 101.981) (width 0.25) (layer F.Cu) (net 9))
 (segment (start 179.785411 103.632) (end 181.689 103.632) (width 0.25) (layer F.Cu) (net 9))
 (segment (start 177.2 105.25) (end 176.751 105.25) (width 0.25) (layer F.Cu) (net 10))
 (segment (start 176.751 105.25) (end 176.403 104.902) (width 0.25) (layer F.Cu) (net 10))
 (segment (start 176.403 104.902) (end 176.403 104.394) (width 0.25) (layer F.Cu) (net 10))
 (segment (start 176.403 104.394) (end 177.6095 103.1875) (width 0.25) (layer F.Cu) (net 10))
 (segment (start 177.6095 103.1875) (end 179.5935 103.1875) (width 0.25) (layer F.Cu) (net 10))
 (segment (start 179.5935 103.1875) (end 180.8 101.981) (width 0.25) (layer F.Cu) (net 10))
 (segment (start 177.927 101.981) (end 178.26 101.981) (width 0.25) (layer F.Cu) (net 11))
 (segment (start 174.117 105.791) (end 177.927 101.981) (width 0.25) (layer F.Cu) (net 11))
 (segment (start 174.117 106.989) (end 174.117 105.791) (width 0.25) (layer F.Cu) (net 11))
 (segment (start 174.628 107.5) (end 174.117 106.989) (width 0.25) (layer F.Cu) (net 11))
 (segment (start 175.75 107.5) (end 174.628 107.5) (width 0.25) (layer F.Cu) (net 11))
 (segment (start 173.435 112.045) (end 173.482 111.998) (width 0.25) (layer F.Cu) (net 14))
 (segment (start 173.435 114.046) (end 173.435 112.045) (width 0.25) (layer F.Cu) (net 14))
 (segment (start 173.784 112.3) (end 173.482 111.998) (width 0.25) (layer F.Cu) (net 14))
 (segment (start 175.75 112.3) (end 173.784 112.3) (width 0.25) (layer F.Cu) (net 14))
 (segment (start 183.584011 104.082011) (end 184.531 105.029) (width 0.25) (layer F.Cu) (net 15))
 (segment (start 180.016989 104.082011) (end 183.584011 104.082011) (width 0.25) (layer F.Cu) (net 15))
 (segment (start 179.6 104.499) (end 180.016989 104.082011) (width 0.25) (layer F.Cu) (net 15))
 (segment (start 179.6 105.25) (end 179.6 104.499) (width 0.25) (layer F.Cu) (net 15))
 (segment (start 181.6 119.83) (end 182.07 120.3) (width 0.25) (layer F.Cu) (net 3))
 (segment (start 181.6 117.5125) (end 181.6 119.83) (width 0.25) (layer F.Cu) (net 3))
 (segment (start 180 119.83) (end 179.53 120.3) (width 0.25) (layer F.Cu) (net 2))
 (segment (start 180 117.5125) (end 180 119.83) (width 0.25) (layer F.Cu) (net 2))
 (segment (start 180.4 115.2875) (end 180.4 113.75) (width 0.25) (layer F.Cu) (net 12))
 (segment (start 180 115.6875) (end 180.4 115.2875) (width 0.25) (layer F.Cu) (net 12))
 (segment (start 181.2 115.2875) (end 181.2 113.75) (width 0.25) (layer F.Cu) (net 13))
 (segment (start 181.6 115.6875) (end 181.2 115.2875) (width 0.25) (layer F.Cu) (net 13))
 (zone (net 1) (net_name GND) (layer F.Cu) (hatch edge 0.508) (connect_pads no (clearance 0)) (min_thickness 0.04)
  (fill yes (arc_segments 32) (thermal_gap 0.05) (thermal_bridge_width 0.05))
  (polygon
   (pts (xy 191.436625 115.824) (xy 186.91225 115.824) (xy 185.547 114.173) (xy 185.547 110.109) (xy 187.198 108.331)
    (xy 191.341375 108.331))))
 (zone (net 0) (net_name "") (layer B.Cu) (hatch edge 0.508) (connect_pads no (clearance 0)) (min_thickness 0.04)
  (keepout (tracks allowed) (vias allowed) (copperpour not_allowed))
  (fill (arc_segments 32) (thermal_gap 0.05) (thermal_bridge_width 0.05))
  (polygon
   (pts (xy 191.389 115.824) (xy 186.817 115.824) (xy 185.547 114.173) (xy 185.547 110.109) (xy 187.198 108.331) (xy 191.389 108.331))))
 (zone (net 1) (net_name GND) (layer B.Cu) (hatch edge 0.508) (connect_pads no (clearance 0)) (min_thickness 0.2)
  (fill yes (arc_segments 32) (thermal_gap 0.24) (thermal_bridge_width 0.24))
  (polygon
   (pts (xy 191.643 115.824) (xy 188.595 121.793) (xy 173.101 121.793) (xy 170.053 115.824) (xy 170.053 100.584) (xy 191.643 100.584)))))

